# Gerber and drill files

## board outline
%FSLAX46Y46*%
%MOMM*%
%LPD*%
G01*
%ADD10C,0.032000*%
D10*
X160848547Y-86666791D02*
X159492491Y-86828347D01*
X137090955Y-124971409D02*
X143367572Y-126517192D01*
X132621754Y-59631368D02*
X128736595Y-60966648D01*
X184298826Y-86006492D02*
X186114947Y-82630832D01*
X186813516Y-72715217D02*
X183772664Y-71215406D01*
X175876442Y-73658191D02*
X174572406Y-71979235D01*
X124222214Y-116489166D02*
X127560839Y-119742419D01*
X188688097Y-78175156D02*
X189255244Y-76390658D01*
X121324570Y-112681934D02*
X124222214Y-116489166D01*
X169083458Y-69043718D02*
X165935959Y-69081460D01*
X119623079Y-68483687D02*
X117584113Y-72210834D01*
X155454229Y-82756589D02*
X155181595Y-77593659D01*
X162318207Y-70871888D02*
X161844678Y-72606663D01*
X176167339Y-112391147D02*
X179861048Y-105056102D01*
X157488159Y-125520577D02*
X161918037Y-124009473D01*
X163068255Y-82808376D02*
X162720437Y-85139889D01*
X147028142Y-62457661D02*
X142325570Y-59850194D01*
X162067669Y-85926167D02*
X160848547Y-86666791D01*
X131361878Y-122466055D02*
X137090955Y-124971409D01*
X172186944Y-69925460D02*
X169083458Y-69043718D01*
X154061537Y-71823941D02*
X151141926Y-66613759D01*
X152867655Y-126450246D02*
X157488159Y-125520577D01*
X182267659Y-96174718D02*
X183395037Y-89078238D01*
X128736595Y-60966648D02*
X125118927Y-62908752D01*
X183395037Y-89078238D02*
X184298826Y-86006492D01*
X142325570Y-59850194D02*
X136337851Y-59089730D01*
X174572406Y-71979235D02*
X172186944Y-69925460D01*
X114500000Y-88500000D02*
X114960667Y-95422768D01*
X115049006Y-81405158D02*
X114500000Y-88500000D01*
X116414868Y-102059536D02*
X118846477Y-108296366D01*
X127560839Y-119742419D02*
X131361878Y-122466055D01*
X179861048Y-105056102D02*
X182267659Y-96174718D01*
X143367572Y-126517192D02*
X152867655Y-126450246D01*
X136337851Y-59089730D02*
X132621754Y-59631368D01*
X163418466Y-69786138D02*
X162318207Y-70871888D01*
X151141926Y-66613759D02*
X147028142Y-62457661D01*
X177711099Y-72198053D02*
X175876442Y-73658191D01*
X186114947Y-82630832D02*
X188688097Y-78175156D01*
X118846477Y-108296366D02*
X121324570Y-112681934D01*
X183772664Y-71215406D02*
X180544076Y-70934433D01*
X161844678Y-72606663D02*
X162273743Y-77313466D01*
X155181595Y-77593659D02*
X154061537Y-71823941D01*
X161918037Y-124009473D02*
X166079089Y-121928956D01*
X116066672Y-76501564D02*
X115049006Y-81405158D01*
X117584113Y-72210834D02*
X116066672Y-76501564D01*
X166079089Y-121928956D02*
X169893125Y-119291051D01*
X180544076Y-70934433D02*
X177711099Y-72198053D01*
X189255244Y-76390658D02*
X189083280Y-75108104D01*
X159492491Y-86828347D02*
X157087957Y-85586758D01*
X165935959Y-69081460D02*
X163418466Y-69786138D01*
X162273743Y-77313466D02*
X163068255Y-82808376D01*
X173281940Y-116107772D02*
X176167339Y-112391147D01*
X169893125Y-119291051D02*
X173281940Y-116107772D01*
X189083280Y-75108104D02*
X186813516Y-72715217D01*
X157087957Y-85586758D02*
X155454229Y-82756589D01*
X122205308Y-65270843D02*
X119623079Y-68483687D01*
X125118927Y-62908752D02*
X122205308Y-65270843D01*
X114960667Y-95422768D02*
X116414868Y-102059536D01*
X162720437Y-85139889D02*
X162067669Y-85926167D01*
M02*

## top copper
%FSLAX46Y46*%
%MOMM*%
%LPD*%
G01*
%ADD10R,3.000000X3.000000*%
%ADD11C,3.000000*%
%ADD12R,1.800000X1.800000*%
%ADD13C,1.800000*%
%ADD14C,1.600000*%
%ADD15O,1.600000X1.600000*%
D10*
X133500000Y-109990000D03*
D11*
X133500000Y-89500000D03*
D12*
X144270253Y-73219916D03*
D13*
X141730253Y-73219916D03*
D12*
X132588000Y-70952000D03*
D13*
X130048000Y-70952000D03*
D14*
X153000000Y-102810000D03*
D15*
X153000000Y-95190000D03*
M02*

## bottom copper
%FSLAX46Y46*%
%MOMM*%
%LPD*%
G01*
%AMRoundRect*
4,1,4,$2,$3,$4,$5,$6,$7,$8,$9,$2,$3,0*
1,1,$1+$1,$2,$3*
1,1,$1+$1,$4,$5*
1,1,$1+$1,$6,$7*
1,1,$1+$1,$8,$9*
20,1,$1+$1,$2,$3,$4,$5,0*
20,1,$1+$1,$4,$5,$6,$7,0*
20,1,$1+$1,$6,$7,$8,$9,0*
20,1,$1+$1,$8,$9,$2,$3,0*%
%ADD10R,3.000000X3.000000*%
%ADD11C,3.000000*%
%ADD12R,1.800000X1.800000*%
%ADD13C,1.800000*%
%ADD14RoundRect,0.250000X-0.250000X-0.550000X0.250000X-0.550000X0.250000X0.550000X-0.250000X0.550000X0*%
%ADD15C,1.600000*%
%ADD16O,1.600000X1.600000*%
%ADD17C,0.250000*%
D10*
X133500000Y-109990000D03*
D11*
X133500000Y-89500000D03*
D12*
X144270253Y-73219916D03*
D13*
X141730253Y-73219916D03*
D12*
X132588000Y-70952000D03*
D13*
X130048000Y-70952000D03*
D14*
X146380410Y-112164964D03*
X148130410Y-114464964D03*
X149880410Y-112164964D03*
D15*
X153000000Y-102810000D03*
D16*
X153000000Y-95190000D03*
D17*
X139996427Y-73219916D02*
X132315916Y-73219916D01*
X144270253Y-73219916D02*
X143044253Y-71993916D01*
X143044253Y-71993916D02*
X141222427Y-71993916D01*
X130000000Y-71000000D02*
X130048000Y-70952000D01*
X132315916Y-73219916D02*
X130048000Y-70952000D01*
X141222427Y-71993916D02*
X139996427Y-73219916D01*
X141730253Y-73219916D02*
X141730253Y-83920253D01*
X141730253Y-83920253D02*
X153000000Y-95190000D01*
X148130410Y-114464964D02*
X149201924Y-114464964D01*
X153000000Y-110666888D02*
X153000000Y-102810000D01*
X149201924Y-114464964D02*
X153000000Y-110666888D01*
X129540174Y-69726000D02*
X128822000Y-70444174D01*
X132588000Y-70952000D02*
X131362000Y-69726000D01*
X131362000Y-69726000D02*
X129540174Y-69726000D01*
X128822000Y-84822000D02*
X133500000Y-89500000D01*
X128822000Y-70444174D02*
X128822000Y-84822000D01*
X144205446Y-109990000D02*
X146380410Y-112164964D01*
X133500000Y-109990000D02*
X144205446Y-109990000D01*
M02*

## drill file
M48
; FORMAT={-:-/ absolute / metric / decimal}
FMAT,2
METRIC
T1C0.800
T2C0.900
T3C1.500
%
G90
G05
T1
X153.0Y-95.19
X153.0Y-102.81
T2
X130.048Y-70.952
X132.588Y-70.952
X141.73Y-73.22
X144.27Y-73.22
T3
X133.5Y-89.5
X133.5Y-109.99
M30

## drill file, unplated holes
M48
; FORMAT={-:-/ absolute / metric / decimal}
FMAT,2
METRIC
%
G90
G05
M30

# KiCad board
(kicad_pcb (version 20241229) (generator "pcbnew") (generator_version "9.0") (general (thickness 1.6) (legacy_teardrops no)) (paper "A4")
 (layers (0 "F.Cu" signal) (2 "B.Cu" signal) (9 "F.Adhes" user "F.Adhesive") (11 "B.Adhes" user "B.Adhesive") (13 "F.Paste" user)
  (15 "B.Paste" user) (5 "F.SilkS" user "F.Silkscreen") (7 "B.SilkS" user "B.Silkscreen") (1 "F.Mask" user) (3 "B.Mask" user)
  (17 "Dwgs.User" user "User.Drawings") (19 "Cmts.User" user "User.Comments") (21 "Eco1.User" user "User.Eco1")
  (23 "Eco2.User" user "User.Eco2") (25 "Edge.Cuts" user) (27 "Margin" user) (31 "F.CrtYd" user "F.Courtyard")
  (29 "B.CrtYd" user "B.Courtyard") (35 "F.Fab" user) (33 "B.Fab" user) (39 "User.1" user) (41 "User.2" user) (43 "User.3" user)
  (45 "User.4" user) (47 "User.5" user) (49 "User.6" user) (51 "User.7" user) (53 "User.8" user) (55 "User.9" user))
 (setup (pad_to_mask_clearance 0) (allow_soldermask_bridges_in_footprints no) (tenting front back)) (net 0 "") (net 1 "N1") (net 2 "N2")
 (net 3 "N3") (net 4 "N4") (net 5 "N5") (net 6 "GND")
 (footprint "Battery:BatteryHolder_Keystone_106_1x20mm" (layer "B.Cu") (at 133.5 109.99 90)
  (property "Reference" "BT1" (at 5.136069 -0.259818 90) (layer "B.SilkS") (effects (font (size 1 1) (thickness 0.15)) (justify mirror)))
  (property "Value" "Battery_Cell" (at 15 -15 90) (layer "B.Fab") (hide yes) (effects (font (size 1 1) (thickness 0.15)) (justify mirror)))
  (pad "1" thru_hole rect (at 0 0 90) (size 3 3) (drill 1.5) (layers "*.Cu" "*.Mask") (remove_unused_layers no) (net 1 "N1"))
  (pad "2" thru_hole circle (at 20.49 0 90) (size 3 3) (drill 1.5) (layers "*.Cu" "*.Mask") (remove_unused_layers no) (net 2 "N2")))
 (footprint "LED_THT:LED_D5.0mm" (layer "B.Cu") (at 144.270253 73.219916 180)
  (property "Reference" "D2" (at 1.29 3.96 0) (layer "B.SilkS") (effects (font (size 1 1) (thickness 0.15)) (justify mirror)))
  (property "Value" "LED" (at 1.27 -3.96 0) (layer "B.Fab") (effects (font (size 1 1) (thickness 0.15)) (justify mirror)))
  (pad "1" thru_hole rect (at 0 0 180) (size 1.8 1.8) (drill 0.9) (layers "*.Cu" "*.Mask") (remove_unused_layers no) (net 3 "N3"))
  (pad "2" thru_hole circle (at 2.54 0 180) (size 1.8 1.8) (drill 0.9) (layers "*.Cu" "*.Mask") (remove_unused_layers no) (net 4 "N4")))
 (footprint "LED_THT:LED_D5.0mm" (layer "B.Cu") (at 132.588 70.952 180)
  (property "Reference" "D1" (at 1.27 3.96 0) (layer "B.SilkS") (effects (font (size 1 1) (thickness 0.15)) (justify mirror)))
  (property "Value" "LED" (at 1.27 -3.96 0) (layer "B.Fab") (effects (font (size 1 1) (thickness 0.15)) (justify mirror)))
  (pad "1" thru_hole rect (at 0 0 180) (size 1.8 1.8) (drill 0.9) (layers "*.Cu" "*.Mask") (remove_unused_layers no) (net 2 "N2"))
  (pad "2" thru_hole circle (at 2.54 0 180) (size 1.8 1.8) (drill 0.9) (layers "*.Cu" "*.Mask") (remove_unused_layers no) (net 3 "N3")))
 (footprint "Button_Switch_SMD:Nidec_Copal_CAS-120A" (layer "B.Cu") (at 148.13041 113.314964 -90)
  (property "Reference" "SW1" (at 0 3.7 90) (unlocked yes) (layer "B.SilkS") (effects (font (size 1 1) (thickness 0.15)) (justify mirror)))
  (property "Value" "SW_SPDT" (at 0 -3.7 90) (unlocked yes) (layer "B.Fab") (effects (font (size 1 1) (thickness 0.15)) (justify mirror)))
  (pad "1" smd roundrect (at -1.15 1.75) (size 1 1.6) (layers "B.Cu" "B.Mask" "B.Paste") (roundrect_rratio 0.25) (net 1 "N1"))
  (pad "2" smd roundrect (at 1.15 0) (size 1 1.6) (layers "B.Cu" "B.Mask" "B.Paste") (roundrect_rratio 0.25) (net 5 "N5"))
  (pad "3" smd roundrect (at -1.15 -1.75) (size 1 1.6) (layers "B.Cu" "B.Mask" "B.Paste") (roundrect_rratio 0.25) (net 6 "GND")))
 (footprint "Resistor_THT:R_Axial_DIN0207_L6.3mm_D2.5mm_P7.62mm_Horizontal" (layer "B.Cu") (at 153 102.81 90)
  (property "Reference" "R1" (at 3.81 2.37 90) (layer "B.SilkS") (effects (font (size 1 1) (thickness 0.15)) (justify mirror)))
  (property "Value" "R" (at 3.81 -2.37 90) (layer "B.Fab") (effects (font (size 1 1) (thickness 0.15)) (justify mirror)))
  (pad "1" thru_hole circle (at 0 0 90) (size 1.6 1.6) (drill 0.8) (layers "*.Cu" "*.Mask") (remove_unused_layers no) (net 5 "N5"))
  (pad "2" thru_hole oval (at 7.62 0 90) (size 1.6 1.6) (drill 0.8) (layers "*.Cu" "*.Mask") (remove_unused_layers no) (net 4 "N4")))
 (gr_line (start 160.848547 86.666791) (end 159.492491 86.828347) (stroke (width 0.032) (type default)) (layer "Edge.Cuts"))
 (gr_line (start 137.090955 124.971409) (end 143.367572 126.517192) (stroke (width 0.032) (type default)) (layer "Edge.Cuts"))
 (gr_line (start 132.621754 59.631368) (end 128.736595 60.966648) (stroke (width 0.032) (type default)) (layer "Edge.Cuts"))
 (gr_line (start 184.298826 86.006492) (end 186.114947 82.630832) (stroke (width 0.032) (type default)) (layer "Edge.Cuts"))
 (gr_line (start 186.813516 72.715217) (end 183.772664 71.215406) (stroke (width 0.032) (type default)) (layer "Edge.Cuts"))
 (gr_line (start 175.876442 73.658191) (end 174.572406 71.979235) (stroke (width 0.032) (type default)) (layer "Edge.Cuts"))
 (gr_line (start 124.222214 116.489166) (end 127.560839 119.742419) (stroke (width 0.032) (type default)) (layer "Edge.Cuts"))
 (gr_line (start 188.688097 78.175156) (end 189.255244 76.390658) (stroke (width 0.032) (type default)) (layer "Edge.Cuts"))
 (gr_line (start 121.32457 112.681934) (end 124.222214 116.489166) (stroke (width 0.032) (type default)) (layer "Edge.Cuts"))
 (gr_line (start 169.083458 69.043718) (end 165.935959 69.08146) (stroke (width 0.032) (type default)) (layer "Edge.Cuts"))
 (gr_line (start 119.623079 68.483687) (end 117.584113 72.210834) (stroke (width 0.032) (type default)) (layer "Edge.Cuts"))
 (gr_line (start 155.454229 82.756589) (end 155.181595 77.593659) (stroke (width 0.032) (type default)) (layer "Edge.Cuts"))
 (gr_line (start 162.318207 70.871888) (end 161.844678 72.606663) (stroke (width 0.032) (type default)) (layer "Edge.Cuts"))
 (gr_line (start 176.167339 112.391147) (end 179.861048 105.056102) (stroke (width 0.032) (type default)) (layer "Edge.Cuts"))
 (gr_line (start 157.488159 125.520577) (end 161.918037 124.009473) (stroke (width 0.032) (type default)) (layer "Edge.Cuts"))
 (gr_line (start 163.068255 82.808376) (end 162.720437 85.139889) (stroke (width 0.032) (type default)) (layer "Edge.Cuts"))
 (gr_line (start 147.028142 62.457661) (end 142.32557 59.850194) (stroke (width 0.032) (type default)) (layer "Edge.Cuts"))
 (gr_line (start 162.067669 85.926167) (end 160.848547 86.666791) (stroke (width 0.032) (type default)) (layer "Edge.Cuts"))
 (gr_line (start 131.361878 122.466055) (end 137.090955 124.971409) (stroke (width 0.032) (type default)) (layer "Edge.Cuts"))
 (gr_line (start 172.186944 69.92546) (end 169.083458 69.043718) (stroke (width 0.032) (type default)) (layer "Edge.Cuts"))
 (gr_line (start 154.061537 71.823941) (end 151.141926 66.613759) (stroke (width 0.032) (type default)) (layer "Edge.Cuts"))
 (gr_line (start 152.867655 126.450246) (end 157.488159 125.520577) (stroke (width 0.032) (type default)) (layer "Edge.Cuts"))
 (gr_line (start 182.267659 96.174718) (end 183.395037 89.078238) (stroke (width 0.032) (type default)) (layer "Edge.Cuts"))
 (gr_line (start 128.736595 60.966648) (end 125.118927 62.908752) (stroke (width 0.032) (type default)) (layer "Edge.Cuts"))
 (gr_line (start 183.395037 89.078238) (end 184.298826 86.006492) (stroke (width 0.032) (type default)) (layer "Edge.Cuts"))
 (gr_line (start 142.32557 59.850194) (end 136.337851 59.08973) (stroke (width 0.032) (type default)) (layer "Edge.Cuts"))
 (gr_line (start 174.572406 71.979235) (end 172.186944 69.92546) (stroke (width 0.032) (type default)) (layer "Edge.Cuts"))
 (gr_line (start 114.5 88.5) (end 114.960667 95.422768) (stroke (width 0.032) (type default)) (layer "Edge.Cuts"))
 (gr_line (start 115.049006 81.405158) (end 114.5 88.5) (stroke (width 0.032) (type default)) (layer "Edge.Cuts"))
 (gr_line (start 116.414868 102.059536) (end 118.846477 108.296366) (stroke (width 0.032) (type default)) (layer "Edge.Cuts"))
 (gr_line (start 127.560839 119.742419) (end 131.361878 122.466055) (stroke (width 0.032) (type default)) (layer "Edge.Cuts"))
 (gr_line (start 179.861048 105.056102) (end 182.267659 96.174718) (stroke (width 0.032) (type default)) (layer "Edge.Cuts"))
 (gr_line (start 143.367572 126.517192) (end 152.867655 126.450246) (stroke (width 0.032) (type default)) (layer "Edge.Cuts"))
 (gr_line (start 136.337851 59.08973) (end 132.621754 59.631368) (stroke (width 0.032) (type default)) (layer "Edge.Cuts"))
 (gr_line (start 163.418466 69.786138) (end 162.318207 70.871888) (stroke (width 0.032) (type default)) (layer "Edge.Cuts"))
 (gr_line (start 151.141926 66.613759) (end 147.028142 62.457661) (stroke (width 0.032) (type default)) (layer "Edge.Cuts"))
 (gr_line (start 177.711099 72.198053) (end 175.876442 73.658191) (stroke (width 0.032) (type default)) (layer "Edge.Cuts"))
 (gr_line (start 186.114947 82.630832) (end 188.688097 78.175156) (stroke (width 0.032) (type default)) (layer "Edge.Cuts"))
 (gr_line (start 118.846477 108.296366) (end 121.32457 112.681934) (stroke (width 0.032) (type default)) (layer "Edge.Cuts"))
 (gr_line (start 183.772664 71.215406) (end 180.544076 70.934433) (stroke (width 0.032) (type default)) (layer "Edge.Cuts"))
 (gr_line (start 161.844678 72.606663) (end 162.273743 77.313466) (stroke (width 0.032) (type default)) (layer "Edge.Cuts"))
 (gr_line (start 155.181595 77.593659) (end 154.061537 71.823941) (stroke (width 0.032) (type default)) (layer "Edge.Cuts"))
 (gr_line (start 161.918037 124.009473) (end 166.079089 121.928956) (stroke (width 0.032) (type default)) (layer "Edge.Cuts"))
 (gr_line (start 116.066672 76.501564) (end 115.049006 81.405158) (stroke (width 0.032) (type default)) (layer "Edge.Cuts"))
 (gr_line (start 117.584113 72.210834) (end 116.066672 76.501564) (stroke (width 0.032) (type default)) (layer "Edge.Cuts"))
 (gr_line (start 166.079089 121.928956) (end 169.893125 119.291051) (stroke (width 0.032) (type default)) (layer "Edge.Cuts"))
 (gr_line (start 180.544076 70.934433) (end 177.711099 72.198053) (stroke (width 0.032) (type default)) (layer "Edge.Cuts"))
 (gr_line (start 189.255244 76.390658) (end 189.08328 75.108104) (stroke (width 0.032) (type default)) (layer "Edge.Cuts"))
 (gr_line (start 159.492491 86.828347) (end 157.087957 85.586758) (stroke (width 0.032) (type default)) (layer "Edge.Cuts"))
 (gr_line (start 165.935959 69.08146) (end 163.418466 69.786138) (stroke (width 0.032) (type default)) (layer "Edge.Cuts"))
 (gr_line (start 162.273743 77.313466) (end 163.068255 82.808376) (stroke (width 0.032) (type default)) (layer "Edge.Cuts"))
 (gr_line (start 173.28194 116.107772) (end 176.167339 112.391147) (stroke (width 0.032) (type default)) (layer "Edge.Cuts"))
 (gr_line (start 169.893125 119.291051) (end 173.28194 116.107772) (stroke (width 0.032) (type default)) (layer "Edge.Cuts"))
 (gr_line (start 189.08328 75.108104) (end 186.813516 72.715217) (stroke (width 0.032) (type default)) (layer "Edge.Cuts"))
 (gr_line (start 157.087957 85.586758) (end 155.454229 82.756589) (stroke (width 0.032) (type default)) (layer "Edge.Cuts"))
 (gr_line (start 122.205308 65.270843) (end 119.623079 68.483687) (stroke (width 0.032) (type default)) (layer "Edge.Cuts"))
 (gr_line (start 125.118927 62.908752) (end 122.205308 65.270843) (stroke (width 0.032) (type default)) (layer "Edge.Cuts"))
 (gr_line (start 114.960667 95.422768) (end 116.414868 102.059536) (stroke (width 0.032) (type default)) (layer "Edge.Cuts"))
 (gr_line (start 162.720437 85.139889) (end 162.067669 85.926167) (stroke (width 0.032) (type default)) (layer "Edge.Cuts"))
 (segment (start 139.996427 73.219916) (end 132.315916 73.219916) (width 0.25) (layer "B.Cu") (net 3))
 (segment (start 144.270253 73.219916) (end 143.044253 71.993916) (width 0.25) (layer "B.Cu") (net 3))
 (segment (start 143.044253 71.993916) (end 141.222427 71.993916) (width 0.25) (layer "B.Cu") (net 3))
 (segment (start 130 71) (end 130.048 70.952) (width 0.25) (layer "B.Cu") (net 3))
 (segment (start 132.315916 73.219916) (end 130.048 70.952) (width 0.25) (layer "B.Cu") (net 3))
 (segment (start 141.222427 71.993916) (end 139.996427 73.219916) (width 0.25) (layer "B.Cu") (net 3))
 (segment (start 141.730253 73.219916) (end 141.730253 83.920253) (width 0.25) (layer "B.Cu") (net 4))
 (segment (start 141.730253 83.920253) (end 153 95.19) (width 0.25) (layer "B.Cu") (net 4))
 (segment (start 148.13041 114.464964) (end 149.201924 114.464964) (width 0.25) (layer "B.Cu") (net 5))
 (segment (start 153 110.666888) (end 153 102.81) (width 0.25) (layer "B.Cu") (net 5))
 (segment (start 149.201924 114.464964) (end 153 110.666888) (width 0.25) (layer "B.Cu") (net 5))
 (segment (start 129.540174 69.726) (end 128.822 70.444174) (width 0.25) (layer "B.Cu") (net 2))
 (segment (start 132.588 70.952) (end 131.362 69.726) (width 0.25) (layer "B.Cu") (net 2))
 (segment (start 131.362 69.726) (end 129.540174 69.726) (width 0.25) (layer "B.Cu") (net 2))
 (segment (start 128.822 84.822) (end 133.5 89.5) (width 0.25) (layer "B.Cu") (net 2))
 (segment (start 128.822 70.444174) (end 128.822 84.822) (width 0.25) (layer "B.Cu") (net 2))
 (segment (start 144.205446 109.99) (end 146.38041 112.164964) (width 0.25) (layer "B.Cu") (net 1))
 (segment (start 133.5 109.99) (end 144.205446 109.99) (width 0.25) (layer "B.Cu") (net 1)))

